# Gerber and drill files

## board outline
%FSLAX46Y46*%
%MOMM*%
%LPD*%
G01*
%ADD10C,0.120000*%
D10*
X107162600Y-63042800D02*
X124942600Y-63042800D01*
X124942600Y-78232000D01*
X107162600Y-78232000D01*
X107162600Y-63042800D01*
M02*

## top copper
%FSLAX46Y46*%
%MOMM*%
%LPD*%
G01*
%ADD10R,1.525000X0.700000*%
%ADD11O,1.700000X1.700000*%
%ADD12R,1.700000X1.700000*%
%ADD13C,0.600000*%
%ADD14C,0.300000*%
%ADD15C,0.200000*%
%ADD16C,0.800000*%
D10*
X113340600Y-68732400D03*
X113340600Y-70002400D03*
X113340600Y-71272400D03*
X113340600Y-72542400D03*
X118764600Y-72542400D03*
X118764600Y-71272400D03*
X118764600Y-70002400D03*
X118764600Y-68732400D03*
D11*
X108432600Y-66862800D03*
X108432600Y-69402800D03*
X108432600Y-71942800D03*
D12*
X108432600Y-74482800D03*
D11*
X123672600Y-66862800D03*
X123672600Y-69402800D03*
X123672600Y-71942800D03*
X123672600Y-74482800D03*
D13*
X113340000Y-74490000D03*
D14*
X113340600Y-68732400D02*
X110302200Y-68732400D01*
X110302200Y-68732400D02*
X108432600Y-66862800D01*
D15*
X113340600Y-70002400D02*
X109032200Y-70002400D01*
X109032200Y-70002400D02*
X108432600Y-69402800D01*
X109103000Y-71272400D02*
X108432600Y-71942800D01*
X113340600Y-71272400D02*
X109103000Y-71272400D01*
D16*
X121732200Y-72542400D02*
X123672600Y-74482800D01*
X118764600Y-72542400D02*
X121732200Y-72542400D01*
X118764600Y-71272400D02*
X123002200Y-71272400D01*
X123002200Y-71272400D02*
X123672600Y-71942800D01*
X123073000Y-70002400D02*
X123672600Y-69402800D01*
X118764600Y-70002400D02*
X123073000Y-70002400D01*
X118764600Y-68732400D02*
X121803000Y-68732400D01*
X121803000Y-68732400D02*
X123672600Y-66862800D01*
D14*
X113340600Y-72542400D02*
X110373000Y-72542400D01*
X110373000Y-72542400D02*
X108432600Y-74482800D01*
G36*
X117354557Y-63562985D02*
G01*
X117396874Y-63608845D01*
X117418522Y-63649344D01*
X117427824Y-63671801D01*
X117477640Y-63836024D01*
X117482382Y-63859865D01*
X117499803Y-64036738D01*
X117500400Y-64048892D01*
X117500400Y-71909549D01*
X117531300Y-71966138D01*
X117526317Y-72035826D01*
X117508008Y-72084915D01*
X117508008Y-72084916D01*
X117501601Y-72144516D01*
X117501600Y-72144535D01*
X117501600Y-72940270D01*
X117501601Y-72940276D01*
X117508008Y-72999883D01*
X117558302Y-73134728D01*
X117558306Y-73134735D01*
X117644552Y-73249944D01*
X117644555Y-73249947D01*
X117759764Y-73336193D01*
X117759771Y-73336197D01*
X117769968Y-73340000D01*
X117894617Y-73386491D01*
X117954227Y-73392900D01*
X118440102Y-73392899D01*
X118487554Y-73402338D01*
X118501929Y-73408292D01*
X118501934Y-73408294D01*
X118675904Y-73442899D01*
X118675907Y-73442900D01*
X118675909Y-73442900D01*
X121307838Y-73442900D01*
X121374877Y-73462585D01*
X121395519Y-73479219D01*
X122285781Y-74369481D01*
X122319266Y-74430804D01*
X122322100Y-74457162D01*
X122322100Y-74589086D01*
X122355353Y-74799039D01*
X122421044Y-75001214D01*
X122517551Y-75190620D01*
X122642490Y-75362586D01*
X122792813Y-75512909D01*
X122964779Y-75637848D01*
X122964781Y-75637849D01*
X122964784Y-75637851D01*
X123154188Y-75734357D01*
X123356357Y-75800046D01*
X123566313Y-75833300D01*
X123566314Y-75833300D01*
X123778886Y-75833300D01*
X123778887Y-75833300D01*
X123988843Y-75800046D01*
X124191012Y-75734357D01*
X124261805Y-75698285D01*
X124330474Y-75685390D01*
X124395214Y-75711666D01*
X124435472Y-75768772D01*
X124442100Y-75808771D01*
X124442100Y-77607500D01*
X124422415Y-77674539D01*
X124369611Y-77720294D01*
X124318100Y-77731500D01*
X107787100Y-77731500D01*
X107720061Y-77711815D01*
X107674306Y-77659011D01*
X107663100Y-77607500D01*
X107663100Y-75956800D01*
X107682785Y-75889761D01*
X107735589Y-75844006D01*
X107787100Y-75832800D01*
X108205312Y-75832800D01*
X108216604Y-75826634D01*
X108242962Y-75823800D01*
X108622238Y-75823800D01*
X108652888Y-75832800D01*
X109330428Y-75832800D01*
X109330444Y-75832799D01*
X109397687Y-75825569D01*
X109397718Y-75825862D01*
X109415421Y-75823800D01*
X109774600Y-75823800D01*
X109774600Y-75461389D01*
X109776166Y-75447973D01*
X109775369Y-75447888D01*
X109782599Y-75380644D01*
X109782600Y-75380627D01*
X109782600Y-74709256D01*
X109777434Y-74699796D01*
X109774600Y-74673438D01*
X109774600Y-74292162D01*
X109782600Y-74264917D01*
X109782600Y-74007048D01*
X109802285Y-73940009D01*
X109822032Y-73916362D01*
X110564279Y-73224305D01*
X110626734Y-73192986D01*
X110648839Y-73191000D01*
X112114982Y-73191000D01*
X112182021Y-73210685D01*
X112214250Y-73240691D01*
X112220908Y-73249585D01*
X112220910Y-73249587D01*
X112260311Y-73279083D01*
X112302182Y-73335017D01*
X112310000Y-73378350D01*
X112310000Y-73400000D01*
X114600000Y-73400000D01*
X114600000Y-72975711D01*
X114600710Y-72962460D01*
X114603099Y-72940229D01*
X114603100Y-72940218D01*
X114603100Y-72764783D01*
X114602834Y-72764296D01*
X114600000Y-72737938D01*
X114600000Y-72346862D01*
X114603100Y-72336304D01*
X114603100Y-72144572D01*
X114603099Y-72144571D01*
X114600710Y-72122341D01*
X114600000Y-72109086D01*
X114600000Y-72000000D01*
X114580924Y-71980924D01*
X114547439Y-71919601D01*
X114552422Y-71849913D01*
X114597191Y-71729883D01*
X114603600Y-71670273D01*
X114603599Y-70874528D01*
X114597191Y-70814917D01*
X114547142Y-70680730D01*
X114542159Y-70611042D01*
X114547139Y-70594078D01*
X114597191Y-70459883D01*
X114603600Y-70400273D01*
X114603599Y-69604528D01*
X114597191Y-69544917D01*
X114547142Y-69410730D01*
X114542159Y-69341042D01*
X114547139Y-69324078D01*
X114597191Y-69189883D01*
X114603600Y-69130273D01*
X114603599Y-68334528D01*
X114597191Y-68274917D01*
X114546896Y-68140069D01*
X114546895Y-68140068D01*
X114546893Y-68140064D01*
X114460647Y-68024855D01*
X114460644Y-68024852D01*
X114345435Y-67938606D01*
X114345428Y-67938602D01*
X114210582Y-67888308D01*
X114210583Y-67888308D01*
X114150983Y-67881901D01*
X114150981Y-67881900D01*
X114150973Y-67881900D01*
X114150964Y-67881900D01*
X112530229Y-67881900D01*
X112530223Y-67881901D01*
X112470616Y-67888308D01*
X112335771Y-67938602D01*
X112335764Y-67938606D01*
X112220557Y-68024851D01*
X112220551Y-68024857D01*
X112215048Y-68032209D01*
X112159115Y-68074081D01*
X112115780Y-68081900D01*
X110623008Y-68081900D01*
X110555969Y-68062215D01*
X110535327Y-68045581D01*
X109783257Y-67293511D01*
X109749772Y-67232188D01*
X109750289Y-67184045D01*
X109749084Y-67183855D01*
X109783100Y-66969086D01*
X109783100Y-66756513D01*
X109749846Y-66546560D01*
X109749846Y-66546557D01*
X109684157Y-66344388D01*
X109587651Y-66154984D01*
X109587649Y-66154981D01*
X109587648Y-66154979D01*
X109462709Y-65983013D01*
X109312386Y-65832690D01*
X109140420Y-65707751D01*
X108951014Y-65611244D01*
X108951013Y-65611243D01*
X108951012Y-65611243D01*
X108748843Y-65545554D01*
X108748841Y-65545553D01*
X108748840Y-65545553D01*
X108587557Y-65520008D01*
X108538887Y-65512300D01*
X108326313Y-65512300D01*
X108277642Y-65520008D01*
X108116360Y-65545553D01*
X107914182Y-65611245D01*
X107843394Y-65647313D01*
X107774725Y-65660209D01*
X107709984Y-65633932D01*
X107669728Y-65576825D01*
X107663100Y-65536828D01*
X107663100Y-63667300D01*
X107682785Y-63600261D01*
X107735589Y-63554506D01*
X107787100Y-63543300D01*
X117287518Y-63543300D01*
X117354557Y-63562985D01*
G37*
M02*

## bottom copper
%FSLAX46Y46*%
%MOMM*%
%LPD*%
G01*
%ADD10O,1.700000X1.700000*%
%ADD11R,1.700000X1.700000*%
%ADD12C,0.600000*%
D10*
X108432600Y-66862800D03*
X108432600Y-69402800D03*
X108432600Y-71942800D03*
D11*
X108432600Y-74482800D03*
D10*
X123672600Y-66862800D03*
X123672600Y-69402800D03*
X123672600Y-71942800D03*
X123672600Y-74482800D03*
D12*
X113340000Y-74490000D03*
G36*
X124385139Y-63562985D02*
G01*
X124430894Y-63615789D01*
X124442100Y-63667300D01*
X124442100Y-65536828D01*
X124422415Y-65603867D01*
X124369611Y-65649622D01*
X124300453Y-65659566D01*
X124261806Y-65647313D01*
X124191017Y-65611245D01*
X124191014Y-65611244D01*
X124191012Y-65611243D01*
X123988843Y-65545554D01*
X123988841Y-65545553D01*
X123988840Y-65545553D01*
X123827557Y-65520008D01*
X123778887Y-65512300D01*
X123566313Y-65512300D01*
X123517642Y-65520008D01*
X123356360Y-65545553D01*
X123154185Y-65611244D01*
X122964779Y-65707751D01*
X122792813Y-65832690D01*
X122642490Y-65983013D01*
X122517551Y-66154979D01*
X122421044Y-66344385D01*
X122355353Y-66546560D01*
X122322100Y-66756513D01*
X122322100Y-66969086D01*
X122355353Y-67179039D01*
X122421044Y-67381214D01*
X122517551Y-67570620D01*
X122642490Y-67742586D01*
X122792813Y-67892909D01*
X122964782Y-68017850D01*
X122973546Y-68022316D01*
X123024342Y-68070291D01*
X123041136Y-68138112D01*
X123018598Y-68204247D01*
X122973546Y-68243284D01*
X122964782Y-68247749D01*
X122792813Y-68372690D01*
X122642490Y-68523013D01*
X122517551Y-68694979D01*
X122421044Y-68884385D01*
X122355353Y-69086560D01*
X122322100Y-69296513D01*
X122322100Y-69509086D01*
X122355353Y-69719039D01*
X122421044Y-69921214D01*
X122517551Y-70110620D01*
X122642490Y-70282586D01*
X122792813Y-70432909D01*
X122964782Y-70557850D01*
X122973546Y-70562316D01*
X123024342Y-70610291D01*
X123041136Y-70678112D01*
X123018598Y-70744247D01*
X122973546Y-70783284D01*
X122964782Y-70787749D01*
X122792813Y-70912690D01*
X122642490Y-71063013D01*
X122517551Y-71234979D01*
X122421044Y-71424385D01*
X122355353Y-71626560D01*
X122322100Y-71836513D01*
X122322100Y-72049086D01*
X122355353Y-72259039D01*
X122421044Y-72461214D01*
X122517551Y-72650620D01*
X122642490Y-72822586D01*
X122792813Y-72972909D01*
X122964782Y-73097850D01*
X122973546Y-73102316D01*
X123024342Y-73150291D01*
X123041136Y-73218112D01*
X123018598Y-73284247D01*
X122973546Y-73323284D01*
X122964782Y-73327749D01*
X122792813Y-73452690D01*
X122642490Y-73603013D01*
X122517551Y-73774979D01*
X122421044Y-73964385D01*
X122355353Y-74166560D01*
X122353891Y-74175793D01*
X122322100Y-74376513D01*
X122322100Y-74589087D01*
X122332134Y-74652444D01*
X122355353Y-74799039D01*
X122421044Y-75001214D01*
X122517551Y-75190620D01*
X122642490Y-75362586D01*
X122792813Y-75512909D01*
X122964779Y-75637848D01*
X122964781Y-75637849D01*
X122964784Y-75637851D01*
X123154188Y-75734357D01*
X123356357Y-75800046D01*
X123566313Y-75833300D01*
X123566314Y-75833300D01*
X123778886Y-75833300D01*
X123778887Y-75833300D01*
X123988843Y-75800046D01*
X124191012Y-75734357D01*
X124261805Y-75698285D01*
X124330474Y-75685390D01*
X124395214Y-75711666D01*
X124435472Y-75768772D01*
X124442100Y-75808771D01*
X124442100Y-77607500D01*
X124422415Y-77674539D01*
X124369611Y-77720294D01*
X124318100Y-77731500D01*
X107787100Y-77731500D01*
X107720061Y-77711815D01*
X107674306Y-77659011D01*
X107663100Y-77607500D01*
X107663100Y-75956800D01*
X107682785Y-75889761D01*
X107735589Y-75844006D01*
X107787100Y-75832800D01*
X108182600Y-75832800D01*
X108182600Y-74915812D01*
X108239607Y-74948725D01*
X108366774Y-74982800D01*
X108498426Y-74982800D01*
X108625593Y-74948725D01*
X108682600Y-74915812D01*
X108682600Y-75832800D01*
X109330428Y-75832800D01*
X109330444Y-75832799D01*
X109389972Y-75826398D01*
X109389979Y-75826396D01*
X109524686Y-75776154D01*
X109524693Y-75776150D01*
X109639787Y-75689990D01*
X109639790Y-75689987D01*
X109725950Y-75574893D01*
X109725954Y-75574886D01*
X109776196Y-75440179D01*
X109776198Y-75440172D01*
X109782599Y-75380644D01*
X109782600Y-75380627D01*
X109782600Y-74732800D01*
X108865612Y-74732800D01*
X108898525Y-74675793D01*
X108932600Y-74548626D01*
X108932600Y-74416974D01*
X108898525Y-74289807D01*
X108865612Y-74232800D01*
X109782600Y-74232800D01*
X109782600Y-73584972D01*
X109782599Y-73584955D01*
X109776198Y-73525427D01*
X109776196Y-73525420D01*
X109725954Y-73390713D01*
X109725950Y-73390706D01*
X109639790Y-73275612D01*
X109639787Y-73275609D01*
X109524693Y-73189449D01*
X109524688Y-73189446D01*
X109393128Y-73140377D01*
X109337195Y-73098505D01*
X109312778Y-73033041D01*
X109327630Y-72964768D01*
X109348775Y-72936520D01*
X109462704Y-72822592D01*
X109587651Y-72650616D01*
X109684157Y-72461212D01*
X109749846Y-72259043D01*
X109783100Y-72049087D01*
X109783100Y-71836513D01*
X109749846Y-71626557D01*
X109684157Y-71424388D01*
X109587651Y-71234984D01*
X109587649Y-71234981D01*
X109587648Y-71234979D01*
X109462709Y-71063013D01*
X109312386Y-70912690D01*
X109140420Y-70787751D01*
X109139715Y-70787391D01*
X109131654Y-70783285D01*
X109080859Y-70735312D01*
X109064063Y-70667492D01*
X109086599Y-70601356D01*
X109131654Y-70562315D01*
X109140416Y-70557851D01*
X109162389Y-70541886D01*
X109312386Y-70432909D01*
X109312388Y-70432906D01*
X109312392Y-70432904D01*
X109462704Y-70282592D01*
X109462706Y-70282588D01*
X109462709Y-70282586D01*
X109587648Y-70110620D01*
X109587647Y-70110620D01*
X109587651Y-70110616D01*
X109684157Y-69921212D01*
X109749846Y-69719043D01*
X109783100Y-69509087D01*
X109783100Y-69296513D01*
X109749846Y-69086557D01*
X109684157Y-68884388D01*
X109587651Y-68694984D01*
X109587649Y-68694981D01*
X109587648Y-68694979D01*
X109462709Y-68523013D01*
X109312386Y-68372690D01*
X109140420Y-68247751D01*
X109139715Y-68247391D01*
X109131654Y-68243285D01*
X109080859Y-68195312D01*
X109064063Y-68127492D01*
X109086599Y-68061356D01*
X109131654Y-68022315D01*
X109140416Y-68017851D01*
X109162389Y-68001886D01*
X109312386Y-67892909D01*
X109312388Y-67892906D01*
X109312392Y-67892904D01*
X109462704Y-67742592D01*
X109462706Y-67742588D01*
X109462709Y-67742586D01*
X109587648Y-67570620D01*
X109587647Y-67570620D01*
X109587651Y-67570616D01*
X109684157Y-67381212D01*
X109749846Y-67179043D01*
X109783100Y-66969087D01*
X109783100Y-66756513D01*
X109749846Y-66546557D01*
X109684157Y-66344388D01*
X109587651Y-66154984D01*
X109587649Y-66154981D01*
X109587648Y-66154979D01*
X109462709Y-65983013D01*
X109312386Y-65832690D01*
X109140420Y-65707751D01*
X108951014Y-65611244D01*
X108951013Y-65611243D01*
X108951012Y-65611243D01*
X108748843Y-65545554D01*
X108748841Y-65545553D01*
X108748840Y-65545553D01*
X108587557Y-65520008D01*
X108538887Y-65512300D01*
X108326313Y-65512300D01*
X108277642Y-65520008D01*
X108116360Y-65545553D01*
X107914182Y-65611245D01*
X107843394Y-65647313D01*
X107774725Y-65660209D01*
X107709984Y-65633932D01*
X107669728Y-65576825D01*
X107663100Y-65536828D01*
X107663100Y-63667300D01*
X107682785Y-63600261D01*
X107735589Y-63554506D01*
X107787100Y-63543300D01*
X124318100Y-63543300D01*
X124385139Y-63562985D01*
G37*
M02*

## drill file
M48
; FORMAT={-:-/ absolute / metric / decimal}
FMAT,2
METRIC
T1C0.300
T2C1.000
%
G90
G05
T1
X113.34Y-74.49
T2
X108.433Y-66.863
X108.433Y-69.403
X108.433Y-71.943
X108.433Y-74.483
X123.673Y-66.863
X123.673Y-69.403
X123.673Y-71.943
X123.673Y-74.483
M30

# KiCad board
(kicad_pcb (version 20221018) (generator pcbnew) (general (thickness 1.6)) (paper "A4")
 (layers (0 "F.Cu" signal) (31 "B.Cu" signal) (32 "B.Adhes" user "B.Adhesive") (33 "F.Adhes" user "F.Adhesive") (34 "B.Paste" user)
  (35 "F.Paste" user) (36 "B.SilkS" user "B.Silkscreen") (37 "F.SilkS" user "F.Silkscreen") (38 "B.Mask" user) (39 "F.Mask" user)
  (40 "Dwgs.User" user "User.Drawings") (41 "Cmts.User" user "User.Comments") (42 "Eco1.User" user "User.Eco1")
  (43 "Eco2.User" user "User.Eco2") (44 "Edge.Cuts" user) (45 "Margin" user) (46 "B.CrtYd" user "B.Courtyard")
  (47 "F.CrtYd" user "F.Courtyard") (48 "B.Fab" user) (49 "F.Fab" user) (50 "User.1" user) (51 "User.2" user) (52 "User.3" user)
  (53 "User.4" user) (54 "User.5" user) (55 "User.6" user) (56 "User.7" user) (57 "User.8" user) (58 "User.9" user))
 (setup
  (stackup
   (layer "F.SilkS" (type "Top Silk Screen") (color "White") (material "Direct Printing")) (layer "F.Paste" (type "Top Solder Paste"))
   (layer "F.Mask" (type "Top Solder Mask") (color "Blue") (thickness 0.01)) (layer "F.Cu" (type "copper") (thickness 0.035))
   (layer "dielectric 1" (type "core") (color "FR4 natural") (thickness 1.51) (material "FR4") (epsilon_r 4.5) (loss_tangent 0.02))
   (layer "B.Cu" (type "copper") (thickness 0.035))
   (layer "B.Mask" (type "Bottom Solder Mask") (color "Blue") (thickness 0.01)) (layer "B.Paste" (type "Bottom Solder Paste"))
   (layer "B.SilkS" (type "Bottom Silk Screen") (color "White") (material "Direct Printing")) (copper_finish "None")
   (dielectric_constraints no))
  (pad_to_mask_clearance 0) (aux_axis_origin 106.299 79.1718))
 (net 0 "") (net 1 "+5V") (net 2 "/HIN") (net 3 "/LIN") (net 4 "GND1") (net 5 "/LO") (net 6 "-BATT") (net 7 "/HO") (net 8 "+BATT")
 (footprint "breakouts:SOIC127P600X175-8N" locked (layer "F.Cu") (at 116.0526 70.6374)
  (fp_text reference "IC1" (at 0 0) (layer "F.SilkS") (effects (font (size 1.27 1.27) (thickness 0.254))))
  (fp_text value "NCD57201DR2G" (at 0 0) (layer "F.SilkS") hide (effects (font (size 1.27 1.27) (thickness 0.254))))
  (pad "1" smd rect locked (at -2.712 -1.905 90) (size 0.7 1.525) (layers "F.Cu" "F.Paste" "F.Mask") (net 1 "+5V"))
  (pad "2" smd rect locked (at -2.712 -0.635 90) (size 0.7 1.525) (layers "F.Cu" "F.Paste" "F.Mask") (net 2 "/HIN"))
  (pad "3" smd rect locked (at -2.712 0.635 90) (size 0.7 1.525) (layers "F.Cu" "F.Paste" "F.Mask") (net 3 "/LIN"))
  (pad "4" smd rect locked (at -2.712 1.905 90) (size 0.7 1.525) (layers "F.Cu" "F.Paste" "F.Mask") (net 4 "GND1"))
  (pad "5" smd rect locked (at 2.712 1.905 90) (size 0.7 1.525) (layers "F.Cu" "F.Paste" "F.Mask") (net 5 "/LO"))
  (pad "6" smd rect locked (at 2.712 0.635 90) (size 0.7 1.525) (layers "F.Cu" "F.Paste" "F.Mask") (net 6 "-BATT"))
  (pad "7" smd rect locked (at 2.712 -0.635 90) (size 0.7 1.525) (layers "F.Cu" "F.Paste" "F.Mask") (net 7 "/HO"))
  (pad "8" smd rect locked (at 2.712 -1.905 90) (size 0.7 1.525) (layers "F.Cu" "F.Paste" "F.Mask") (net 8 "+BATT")))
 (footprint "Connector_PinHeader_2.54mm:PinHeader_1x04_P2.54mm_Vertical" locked (layer "B.Cu") (at 108.4326 66.8628 180)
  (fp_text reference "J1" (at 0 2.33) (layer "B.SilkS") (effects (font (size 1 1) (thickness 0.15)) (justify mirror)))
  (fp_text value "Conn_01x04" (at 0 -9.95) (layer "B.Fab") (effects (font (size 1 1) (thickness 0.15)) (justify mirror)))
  (pad "1" thru_hole oval locked (at 0 0 180) (size 1.7 1.7) (drill 1) (layers "*.Cu" "*.Mask") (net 1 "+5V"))
  (pad "2" thru_hole oval locked (at 0 -2.54 180) (size 1.7 1.7) (drill 1) (layers "*.Cu" "*.Mask") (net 2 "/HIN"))
  (pad "3" thru_hole oval locked (at 0 -5.08 180) (size 1.7 1.7) (drill 1) (layers "*.Cu" "*.Mask") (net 3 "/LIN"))
  (pad "4" thru_hole rect locked (at 0 -7.62 180) (size 1.7 1.7) (drill 1) (layers "*.Cu" "*.Mask") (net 4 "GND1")))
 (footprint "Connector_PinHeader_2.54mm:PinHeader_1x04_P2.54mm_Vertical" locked (layer "B.Cu") (at 123.6726 66.8628 180)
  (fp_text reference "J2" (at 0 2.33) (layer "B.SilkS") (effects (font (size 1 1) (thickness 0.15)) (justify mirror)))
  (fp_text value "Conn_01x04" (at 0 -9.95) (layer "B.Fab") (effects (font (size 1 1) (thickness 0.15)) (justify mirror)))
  (pad "1" thru_hole oval locked (at 0 0 180) (size 1.7 1.7) (drill 1) (layers "*.Cu" "*.Mask") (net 8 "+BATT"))
  (pad "2" thru_hole oval locked (at 0 -2.54 180) (size 1.7 1.7) (drill 1) (layers "*.Cu" "*.Mask") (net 7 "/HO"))
  (pad "3" thru_hole oval locked (at 0 -5.08 180) (size 1.7 1.7) (drill 1) (layers "*.Cu" "*.Mask") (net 6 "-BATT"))
  (pad "4" thru_hole oval locked (at 0 -7.62 180) (size 1.7 1.7) (drill 1) (layers "*.Cu" "*.Mask") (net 5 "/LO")))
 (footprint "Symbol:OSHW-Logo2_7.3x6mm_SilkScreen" (layer "B.Cu") (at 116.08 74.99 180)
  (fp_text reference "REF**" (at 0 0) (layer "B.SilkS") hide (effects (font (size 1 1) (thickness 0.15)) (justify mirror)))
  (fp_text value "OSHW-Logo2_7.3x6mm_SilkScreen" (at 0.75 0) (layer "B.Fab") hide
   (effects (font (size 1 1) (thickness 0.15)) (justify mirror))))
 (gr_rect locked (start 107.1626 63.0428) (end 124.9426 78.232) (stroke (width 0.12) (type default)) (fill none) (layer "Edge.Cuts"))
 (segment (start 113.3406 68.7324) (end 110.3022 68.7324) (width 0.3) (layer "F.Cu") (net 1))
 (segment (start 110.3022 68.7324) (end 108.4326 66.8628) (width 0.3) (layer "F.Cu") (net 1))
 (segment (start 113.3406 70.0024) (end 109.0322 70.0024) (width 0.2) (layer "F.Cu") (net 2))
 (segment (start 109.0322 70.0024) (end 108.4326 69.4028) (width 0.2) (layer "F.Cu") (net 2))
 (segment (start 109.103 71.2724) (end 108.4326 71.9428) (width 0.2) (layer "F.Cu") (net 3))
 (segment (start 113.3406 71.2724) (end 109.103 71.2724) (width 0.2) (layer "F.Cu") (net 3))
 (segment (start 121.7322 72.5424) (end 123.6726 74.4828) (width 0.8) (layer "F.Cu") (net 5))
 (segment (start 118.7646 72.5424) (end 121.7322 72.5424) (width 0.8) (layer "F.Cu") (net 5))
 (segment (start 118.7646 71.2724) (end 123.0022 71.2724) (width 0.8) (layer "F.Cu") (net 6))
 (segment (start 123.0022 71.2724) (end 123.6726 71.9428) (width 0.8) (layer "F.Cu") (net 6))
 (segment (start 123.073 70.0024) (end 123.6726 69.4028) (width 0.8) (layer "F.Cu") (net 7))
 (segment (start 118.7646 70.0024) (end 123.073 70.0024) (width 0.8) (layer "F.Cu") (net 7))
 (segment (start 118.7646 68.7324) (end 121.803 68.7324) (width 0.8) (layer "F.Cu") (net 8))
 (segment (start 121.803 68.7324) (end 123.6726 66.8628) (width 0.8) (layer "F.Cu") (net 8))
 (segment (start 113.3406 72.5424) (end 110.373 72.5424) (width 0.3) (layer "F.Cu") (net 4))
 (segment (start 110.373 72.5424) (end 108.4326 74.4828) (width 0.3) (layer "F.Cu") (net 4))
 (via (at 113.34 74.49) (size 0.6) (drill 0.3) (layers "F.Cu" "B.Cu") (free) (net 4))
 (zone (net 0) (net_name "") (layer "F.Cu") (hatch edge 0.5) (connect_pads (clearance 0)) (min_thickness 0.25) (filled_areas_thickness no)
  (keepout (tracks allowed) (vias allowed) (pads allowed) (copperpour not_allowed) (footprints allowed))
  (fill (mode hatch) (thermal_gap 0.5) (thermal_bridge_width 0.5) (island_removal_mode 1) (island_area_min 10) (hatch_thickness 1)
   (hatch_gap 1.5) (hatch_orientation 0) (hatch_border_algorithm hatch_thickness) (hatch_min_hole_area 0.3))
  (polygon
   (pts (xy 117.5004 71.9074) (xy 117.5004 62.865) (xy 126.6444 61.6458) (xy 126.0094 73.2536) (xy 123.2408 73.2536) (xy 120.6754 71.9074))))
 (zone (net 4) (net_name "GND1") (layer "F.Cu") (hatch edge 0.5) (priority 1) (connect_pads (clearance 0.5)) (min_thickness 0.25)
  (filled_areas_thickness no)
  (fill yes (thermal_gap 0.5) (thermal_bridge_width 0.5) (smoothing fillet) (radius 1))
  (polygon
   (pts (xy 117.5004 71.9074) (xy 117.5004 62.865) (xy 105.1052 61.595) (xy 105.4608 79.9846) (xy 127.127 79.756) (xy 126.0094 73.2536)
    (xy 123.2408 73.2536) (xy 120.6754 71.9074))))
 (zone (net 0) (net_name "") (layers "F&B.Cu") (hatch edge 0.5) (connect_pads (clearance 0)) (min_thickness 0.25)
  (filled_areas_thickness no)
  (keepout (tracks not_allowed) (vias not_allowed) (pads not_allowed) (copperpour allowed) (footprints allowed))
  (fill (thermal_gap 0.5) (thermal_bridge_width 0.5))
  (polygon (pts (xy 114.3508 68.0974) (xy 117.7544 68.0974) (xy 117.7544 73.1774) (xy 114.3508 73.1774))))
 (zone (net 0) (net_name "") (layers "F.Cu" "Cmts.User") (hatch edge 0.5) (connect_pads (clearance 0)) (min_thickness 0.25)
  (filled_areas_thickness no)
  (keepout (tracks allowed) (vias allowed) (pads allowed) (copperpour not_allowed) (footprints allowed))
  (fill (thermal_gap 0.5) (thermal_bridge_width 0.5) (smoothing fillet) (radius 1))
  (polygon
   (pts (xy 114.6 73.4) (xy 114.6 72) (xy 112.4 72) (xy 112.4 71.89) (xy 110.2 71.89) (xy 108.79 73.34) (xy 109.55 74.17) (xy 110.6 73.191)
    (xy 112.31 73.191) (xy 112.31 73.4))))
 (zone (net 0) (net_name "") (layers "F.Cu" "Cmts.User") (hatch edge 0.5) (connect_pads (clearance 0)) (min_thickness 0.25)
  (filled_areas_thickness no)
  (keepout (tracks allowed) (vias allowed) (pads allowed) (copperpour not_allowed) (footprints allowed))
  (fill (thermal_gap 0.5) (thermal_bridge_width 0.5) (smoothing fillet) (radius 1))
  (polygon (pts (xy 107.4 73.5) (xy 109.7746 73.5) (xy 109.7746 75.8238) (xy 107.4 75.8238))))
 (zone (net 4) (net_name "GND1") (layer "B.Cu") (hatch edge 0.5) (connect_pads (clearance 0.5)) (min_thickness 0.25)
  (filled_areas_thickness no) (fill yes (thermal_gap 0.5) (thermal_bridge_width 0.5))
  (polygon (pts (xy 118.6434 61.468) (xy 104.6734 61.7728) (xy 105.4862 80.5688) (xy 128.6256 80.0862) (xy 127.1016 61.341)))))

